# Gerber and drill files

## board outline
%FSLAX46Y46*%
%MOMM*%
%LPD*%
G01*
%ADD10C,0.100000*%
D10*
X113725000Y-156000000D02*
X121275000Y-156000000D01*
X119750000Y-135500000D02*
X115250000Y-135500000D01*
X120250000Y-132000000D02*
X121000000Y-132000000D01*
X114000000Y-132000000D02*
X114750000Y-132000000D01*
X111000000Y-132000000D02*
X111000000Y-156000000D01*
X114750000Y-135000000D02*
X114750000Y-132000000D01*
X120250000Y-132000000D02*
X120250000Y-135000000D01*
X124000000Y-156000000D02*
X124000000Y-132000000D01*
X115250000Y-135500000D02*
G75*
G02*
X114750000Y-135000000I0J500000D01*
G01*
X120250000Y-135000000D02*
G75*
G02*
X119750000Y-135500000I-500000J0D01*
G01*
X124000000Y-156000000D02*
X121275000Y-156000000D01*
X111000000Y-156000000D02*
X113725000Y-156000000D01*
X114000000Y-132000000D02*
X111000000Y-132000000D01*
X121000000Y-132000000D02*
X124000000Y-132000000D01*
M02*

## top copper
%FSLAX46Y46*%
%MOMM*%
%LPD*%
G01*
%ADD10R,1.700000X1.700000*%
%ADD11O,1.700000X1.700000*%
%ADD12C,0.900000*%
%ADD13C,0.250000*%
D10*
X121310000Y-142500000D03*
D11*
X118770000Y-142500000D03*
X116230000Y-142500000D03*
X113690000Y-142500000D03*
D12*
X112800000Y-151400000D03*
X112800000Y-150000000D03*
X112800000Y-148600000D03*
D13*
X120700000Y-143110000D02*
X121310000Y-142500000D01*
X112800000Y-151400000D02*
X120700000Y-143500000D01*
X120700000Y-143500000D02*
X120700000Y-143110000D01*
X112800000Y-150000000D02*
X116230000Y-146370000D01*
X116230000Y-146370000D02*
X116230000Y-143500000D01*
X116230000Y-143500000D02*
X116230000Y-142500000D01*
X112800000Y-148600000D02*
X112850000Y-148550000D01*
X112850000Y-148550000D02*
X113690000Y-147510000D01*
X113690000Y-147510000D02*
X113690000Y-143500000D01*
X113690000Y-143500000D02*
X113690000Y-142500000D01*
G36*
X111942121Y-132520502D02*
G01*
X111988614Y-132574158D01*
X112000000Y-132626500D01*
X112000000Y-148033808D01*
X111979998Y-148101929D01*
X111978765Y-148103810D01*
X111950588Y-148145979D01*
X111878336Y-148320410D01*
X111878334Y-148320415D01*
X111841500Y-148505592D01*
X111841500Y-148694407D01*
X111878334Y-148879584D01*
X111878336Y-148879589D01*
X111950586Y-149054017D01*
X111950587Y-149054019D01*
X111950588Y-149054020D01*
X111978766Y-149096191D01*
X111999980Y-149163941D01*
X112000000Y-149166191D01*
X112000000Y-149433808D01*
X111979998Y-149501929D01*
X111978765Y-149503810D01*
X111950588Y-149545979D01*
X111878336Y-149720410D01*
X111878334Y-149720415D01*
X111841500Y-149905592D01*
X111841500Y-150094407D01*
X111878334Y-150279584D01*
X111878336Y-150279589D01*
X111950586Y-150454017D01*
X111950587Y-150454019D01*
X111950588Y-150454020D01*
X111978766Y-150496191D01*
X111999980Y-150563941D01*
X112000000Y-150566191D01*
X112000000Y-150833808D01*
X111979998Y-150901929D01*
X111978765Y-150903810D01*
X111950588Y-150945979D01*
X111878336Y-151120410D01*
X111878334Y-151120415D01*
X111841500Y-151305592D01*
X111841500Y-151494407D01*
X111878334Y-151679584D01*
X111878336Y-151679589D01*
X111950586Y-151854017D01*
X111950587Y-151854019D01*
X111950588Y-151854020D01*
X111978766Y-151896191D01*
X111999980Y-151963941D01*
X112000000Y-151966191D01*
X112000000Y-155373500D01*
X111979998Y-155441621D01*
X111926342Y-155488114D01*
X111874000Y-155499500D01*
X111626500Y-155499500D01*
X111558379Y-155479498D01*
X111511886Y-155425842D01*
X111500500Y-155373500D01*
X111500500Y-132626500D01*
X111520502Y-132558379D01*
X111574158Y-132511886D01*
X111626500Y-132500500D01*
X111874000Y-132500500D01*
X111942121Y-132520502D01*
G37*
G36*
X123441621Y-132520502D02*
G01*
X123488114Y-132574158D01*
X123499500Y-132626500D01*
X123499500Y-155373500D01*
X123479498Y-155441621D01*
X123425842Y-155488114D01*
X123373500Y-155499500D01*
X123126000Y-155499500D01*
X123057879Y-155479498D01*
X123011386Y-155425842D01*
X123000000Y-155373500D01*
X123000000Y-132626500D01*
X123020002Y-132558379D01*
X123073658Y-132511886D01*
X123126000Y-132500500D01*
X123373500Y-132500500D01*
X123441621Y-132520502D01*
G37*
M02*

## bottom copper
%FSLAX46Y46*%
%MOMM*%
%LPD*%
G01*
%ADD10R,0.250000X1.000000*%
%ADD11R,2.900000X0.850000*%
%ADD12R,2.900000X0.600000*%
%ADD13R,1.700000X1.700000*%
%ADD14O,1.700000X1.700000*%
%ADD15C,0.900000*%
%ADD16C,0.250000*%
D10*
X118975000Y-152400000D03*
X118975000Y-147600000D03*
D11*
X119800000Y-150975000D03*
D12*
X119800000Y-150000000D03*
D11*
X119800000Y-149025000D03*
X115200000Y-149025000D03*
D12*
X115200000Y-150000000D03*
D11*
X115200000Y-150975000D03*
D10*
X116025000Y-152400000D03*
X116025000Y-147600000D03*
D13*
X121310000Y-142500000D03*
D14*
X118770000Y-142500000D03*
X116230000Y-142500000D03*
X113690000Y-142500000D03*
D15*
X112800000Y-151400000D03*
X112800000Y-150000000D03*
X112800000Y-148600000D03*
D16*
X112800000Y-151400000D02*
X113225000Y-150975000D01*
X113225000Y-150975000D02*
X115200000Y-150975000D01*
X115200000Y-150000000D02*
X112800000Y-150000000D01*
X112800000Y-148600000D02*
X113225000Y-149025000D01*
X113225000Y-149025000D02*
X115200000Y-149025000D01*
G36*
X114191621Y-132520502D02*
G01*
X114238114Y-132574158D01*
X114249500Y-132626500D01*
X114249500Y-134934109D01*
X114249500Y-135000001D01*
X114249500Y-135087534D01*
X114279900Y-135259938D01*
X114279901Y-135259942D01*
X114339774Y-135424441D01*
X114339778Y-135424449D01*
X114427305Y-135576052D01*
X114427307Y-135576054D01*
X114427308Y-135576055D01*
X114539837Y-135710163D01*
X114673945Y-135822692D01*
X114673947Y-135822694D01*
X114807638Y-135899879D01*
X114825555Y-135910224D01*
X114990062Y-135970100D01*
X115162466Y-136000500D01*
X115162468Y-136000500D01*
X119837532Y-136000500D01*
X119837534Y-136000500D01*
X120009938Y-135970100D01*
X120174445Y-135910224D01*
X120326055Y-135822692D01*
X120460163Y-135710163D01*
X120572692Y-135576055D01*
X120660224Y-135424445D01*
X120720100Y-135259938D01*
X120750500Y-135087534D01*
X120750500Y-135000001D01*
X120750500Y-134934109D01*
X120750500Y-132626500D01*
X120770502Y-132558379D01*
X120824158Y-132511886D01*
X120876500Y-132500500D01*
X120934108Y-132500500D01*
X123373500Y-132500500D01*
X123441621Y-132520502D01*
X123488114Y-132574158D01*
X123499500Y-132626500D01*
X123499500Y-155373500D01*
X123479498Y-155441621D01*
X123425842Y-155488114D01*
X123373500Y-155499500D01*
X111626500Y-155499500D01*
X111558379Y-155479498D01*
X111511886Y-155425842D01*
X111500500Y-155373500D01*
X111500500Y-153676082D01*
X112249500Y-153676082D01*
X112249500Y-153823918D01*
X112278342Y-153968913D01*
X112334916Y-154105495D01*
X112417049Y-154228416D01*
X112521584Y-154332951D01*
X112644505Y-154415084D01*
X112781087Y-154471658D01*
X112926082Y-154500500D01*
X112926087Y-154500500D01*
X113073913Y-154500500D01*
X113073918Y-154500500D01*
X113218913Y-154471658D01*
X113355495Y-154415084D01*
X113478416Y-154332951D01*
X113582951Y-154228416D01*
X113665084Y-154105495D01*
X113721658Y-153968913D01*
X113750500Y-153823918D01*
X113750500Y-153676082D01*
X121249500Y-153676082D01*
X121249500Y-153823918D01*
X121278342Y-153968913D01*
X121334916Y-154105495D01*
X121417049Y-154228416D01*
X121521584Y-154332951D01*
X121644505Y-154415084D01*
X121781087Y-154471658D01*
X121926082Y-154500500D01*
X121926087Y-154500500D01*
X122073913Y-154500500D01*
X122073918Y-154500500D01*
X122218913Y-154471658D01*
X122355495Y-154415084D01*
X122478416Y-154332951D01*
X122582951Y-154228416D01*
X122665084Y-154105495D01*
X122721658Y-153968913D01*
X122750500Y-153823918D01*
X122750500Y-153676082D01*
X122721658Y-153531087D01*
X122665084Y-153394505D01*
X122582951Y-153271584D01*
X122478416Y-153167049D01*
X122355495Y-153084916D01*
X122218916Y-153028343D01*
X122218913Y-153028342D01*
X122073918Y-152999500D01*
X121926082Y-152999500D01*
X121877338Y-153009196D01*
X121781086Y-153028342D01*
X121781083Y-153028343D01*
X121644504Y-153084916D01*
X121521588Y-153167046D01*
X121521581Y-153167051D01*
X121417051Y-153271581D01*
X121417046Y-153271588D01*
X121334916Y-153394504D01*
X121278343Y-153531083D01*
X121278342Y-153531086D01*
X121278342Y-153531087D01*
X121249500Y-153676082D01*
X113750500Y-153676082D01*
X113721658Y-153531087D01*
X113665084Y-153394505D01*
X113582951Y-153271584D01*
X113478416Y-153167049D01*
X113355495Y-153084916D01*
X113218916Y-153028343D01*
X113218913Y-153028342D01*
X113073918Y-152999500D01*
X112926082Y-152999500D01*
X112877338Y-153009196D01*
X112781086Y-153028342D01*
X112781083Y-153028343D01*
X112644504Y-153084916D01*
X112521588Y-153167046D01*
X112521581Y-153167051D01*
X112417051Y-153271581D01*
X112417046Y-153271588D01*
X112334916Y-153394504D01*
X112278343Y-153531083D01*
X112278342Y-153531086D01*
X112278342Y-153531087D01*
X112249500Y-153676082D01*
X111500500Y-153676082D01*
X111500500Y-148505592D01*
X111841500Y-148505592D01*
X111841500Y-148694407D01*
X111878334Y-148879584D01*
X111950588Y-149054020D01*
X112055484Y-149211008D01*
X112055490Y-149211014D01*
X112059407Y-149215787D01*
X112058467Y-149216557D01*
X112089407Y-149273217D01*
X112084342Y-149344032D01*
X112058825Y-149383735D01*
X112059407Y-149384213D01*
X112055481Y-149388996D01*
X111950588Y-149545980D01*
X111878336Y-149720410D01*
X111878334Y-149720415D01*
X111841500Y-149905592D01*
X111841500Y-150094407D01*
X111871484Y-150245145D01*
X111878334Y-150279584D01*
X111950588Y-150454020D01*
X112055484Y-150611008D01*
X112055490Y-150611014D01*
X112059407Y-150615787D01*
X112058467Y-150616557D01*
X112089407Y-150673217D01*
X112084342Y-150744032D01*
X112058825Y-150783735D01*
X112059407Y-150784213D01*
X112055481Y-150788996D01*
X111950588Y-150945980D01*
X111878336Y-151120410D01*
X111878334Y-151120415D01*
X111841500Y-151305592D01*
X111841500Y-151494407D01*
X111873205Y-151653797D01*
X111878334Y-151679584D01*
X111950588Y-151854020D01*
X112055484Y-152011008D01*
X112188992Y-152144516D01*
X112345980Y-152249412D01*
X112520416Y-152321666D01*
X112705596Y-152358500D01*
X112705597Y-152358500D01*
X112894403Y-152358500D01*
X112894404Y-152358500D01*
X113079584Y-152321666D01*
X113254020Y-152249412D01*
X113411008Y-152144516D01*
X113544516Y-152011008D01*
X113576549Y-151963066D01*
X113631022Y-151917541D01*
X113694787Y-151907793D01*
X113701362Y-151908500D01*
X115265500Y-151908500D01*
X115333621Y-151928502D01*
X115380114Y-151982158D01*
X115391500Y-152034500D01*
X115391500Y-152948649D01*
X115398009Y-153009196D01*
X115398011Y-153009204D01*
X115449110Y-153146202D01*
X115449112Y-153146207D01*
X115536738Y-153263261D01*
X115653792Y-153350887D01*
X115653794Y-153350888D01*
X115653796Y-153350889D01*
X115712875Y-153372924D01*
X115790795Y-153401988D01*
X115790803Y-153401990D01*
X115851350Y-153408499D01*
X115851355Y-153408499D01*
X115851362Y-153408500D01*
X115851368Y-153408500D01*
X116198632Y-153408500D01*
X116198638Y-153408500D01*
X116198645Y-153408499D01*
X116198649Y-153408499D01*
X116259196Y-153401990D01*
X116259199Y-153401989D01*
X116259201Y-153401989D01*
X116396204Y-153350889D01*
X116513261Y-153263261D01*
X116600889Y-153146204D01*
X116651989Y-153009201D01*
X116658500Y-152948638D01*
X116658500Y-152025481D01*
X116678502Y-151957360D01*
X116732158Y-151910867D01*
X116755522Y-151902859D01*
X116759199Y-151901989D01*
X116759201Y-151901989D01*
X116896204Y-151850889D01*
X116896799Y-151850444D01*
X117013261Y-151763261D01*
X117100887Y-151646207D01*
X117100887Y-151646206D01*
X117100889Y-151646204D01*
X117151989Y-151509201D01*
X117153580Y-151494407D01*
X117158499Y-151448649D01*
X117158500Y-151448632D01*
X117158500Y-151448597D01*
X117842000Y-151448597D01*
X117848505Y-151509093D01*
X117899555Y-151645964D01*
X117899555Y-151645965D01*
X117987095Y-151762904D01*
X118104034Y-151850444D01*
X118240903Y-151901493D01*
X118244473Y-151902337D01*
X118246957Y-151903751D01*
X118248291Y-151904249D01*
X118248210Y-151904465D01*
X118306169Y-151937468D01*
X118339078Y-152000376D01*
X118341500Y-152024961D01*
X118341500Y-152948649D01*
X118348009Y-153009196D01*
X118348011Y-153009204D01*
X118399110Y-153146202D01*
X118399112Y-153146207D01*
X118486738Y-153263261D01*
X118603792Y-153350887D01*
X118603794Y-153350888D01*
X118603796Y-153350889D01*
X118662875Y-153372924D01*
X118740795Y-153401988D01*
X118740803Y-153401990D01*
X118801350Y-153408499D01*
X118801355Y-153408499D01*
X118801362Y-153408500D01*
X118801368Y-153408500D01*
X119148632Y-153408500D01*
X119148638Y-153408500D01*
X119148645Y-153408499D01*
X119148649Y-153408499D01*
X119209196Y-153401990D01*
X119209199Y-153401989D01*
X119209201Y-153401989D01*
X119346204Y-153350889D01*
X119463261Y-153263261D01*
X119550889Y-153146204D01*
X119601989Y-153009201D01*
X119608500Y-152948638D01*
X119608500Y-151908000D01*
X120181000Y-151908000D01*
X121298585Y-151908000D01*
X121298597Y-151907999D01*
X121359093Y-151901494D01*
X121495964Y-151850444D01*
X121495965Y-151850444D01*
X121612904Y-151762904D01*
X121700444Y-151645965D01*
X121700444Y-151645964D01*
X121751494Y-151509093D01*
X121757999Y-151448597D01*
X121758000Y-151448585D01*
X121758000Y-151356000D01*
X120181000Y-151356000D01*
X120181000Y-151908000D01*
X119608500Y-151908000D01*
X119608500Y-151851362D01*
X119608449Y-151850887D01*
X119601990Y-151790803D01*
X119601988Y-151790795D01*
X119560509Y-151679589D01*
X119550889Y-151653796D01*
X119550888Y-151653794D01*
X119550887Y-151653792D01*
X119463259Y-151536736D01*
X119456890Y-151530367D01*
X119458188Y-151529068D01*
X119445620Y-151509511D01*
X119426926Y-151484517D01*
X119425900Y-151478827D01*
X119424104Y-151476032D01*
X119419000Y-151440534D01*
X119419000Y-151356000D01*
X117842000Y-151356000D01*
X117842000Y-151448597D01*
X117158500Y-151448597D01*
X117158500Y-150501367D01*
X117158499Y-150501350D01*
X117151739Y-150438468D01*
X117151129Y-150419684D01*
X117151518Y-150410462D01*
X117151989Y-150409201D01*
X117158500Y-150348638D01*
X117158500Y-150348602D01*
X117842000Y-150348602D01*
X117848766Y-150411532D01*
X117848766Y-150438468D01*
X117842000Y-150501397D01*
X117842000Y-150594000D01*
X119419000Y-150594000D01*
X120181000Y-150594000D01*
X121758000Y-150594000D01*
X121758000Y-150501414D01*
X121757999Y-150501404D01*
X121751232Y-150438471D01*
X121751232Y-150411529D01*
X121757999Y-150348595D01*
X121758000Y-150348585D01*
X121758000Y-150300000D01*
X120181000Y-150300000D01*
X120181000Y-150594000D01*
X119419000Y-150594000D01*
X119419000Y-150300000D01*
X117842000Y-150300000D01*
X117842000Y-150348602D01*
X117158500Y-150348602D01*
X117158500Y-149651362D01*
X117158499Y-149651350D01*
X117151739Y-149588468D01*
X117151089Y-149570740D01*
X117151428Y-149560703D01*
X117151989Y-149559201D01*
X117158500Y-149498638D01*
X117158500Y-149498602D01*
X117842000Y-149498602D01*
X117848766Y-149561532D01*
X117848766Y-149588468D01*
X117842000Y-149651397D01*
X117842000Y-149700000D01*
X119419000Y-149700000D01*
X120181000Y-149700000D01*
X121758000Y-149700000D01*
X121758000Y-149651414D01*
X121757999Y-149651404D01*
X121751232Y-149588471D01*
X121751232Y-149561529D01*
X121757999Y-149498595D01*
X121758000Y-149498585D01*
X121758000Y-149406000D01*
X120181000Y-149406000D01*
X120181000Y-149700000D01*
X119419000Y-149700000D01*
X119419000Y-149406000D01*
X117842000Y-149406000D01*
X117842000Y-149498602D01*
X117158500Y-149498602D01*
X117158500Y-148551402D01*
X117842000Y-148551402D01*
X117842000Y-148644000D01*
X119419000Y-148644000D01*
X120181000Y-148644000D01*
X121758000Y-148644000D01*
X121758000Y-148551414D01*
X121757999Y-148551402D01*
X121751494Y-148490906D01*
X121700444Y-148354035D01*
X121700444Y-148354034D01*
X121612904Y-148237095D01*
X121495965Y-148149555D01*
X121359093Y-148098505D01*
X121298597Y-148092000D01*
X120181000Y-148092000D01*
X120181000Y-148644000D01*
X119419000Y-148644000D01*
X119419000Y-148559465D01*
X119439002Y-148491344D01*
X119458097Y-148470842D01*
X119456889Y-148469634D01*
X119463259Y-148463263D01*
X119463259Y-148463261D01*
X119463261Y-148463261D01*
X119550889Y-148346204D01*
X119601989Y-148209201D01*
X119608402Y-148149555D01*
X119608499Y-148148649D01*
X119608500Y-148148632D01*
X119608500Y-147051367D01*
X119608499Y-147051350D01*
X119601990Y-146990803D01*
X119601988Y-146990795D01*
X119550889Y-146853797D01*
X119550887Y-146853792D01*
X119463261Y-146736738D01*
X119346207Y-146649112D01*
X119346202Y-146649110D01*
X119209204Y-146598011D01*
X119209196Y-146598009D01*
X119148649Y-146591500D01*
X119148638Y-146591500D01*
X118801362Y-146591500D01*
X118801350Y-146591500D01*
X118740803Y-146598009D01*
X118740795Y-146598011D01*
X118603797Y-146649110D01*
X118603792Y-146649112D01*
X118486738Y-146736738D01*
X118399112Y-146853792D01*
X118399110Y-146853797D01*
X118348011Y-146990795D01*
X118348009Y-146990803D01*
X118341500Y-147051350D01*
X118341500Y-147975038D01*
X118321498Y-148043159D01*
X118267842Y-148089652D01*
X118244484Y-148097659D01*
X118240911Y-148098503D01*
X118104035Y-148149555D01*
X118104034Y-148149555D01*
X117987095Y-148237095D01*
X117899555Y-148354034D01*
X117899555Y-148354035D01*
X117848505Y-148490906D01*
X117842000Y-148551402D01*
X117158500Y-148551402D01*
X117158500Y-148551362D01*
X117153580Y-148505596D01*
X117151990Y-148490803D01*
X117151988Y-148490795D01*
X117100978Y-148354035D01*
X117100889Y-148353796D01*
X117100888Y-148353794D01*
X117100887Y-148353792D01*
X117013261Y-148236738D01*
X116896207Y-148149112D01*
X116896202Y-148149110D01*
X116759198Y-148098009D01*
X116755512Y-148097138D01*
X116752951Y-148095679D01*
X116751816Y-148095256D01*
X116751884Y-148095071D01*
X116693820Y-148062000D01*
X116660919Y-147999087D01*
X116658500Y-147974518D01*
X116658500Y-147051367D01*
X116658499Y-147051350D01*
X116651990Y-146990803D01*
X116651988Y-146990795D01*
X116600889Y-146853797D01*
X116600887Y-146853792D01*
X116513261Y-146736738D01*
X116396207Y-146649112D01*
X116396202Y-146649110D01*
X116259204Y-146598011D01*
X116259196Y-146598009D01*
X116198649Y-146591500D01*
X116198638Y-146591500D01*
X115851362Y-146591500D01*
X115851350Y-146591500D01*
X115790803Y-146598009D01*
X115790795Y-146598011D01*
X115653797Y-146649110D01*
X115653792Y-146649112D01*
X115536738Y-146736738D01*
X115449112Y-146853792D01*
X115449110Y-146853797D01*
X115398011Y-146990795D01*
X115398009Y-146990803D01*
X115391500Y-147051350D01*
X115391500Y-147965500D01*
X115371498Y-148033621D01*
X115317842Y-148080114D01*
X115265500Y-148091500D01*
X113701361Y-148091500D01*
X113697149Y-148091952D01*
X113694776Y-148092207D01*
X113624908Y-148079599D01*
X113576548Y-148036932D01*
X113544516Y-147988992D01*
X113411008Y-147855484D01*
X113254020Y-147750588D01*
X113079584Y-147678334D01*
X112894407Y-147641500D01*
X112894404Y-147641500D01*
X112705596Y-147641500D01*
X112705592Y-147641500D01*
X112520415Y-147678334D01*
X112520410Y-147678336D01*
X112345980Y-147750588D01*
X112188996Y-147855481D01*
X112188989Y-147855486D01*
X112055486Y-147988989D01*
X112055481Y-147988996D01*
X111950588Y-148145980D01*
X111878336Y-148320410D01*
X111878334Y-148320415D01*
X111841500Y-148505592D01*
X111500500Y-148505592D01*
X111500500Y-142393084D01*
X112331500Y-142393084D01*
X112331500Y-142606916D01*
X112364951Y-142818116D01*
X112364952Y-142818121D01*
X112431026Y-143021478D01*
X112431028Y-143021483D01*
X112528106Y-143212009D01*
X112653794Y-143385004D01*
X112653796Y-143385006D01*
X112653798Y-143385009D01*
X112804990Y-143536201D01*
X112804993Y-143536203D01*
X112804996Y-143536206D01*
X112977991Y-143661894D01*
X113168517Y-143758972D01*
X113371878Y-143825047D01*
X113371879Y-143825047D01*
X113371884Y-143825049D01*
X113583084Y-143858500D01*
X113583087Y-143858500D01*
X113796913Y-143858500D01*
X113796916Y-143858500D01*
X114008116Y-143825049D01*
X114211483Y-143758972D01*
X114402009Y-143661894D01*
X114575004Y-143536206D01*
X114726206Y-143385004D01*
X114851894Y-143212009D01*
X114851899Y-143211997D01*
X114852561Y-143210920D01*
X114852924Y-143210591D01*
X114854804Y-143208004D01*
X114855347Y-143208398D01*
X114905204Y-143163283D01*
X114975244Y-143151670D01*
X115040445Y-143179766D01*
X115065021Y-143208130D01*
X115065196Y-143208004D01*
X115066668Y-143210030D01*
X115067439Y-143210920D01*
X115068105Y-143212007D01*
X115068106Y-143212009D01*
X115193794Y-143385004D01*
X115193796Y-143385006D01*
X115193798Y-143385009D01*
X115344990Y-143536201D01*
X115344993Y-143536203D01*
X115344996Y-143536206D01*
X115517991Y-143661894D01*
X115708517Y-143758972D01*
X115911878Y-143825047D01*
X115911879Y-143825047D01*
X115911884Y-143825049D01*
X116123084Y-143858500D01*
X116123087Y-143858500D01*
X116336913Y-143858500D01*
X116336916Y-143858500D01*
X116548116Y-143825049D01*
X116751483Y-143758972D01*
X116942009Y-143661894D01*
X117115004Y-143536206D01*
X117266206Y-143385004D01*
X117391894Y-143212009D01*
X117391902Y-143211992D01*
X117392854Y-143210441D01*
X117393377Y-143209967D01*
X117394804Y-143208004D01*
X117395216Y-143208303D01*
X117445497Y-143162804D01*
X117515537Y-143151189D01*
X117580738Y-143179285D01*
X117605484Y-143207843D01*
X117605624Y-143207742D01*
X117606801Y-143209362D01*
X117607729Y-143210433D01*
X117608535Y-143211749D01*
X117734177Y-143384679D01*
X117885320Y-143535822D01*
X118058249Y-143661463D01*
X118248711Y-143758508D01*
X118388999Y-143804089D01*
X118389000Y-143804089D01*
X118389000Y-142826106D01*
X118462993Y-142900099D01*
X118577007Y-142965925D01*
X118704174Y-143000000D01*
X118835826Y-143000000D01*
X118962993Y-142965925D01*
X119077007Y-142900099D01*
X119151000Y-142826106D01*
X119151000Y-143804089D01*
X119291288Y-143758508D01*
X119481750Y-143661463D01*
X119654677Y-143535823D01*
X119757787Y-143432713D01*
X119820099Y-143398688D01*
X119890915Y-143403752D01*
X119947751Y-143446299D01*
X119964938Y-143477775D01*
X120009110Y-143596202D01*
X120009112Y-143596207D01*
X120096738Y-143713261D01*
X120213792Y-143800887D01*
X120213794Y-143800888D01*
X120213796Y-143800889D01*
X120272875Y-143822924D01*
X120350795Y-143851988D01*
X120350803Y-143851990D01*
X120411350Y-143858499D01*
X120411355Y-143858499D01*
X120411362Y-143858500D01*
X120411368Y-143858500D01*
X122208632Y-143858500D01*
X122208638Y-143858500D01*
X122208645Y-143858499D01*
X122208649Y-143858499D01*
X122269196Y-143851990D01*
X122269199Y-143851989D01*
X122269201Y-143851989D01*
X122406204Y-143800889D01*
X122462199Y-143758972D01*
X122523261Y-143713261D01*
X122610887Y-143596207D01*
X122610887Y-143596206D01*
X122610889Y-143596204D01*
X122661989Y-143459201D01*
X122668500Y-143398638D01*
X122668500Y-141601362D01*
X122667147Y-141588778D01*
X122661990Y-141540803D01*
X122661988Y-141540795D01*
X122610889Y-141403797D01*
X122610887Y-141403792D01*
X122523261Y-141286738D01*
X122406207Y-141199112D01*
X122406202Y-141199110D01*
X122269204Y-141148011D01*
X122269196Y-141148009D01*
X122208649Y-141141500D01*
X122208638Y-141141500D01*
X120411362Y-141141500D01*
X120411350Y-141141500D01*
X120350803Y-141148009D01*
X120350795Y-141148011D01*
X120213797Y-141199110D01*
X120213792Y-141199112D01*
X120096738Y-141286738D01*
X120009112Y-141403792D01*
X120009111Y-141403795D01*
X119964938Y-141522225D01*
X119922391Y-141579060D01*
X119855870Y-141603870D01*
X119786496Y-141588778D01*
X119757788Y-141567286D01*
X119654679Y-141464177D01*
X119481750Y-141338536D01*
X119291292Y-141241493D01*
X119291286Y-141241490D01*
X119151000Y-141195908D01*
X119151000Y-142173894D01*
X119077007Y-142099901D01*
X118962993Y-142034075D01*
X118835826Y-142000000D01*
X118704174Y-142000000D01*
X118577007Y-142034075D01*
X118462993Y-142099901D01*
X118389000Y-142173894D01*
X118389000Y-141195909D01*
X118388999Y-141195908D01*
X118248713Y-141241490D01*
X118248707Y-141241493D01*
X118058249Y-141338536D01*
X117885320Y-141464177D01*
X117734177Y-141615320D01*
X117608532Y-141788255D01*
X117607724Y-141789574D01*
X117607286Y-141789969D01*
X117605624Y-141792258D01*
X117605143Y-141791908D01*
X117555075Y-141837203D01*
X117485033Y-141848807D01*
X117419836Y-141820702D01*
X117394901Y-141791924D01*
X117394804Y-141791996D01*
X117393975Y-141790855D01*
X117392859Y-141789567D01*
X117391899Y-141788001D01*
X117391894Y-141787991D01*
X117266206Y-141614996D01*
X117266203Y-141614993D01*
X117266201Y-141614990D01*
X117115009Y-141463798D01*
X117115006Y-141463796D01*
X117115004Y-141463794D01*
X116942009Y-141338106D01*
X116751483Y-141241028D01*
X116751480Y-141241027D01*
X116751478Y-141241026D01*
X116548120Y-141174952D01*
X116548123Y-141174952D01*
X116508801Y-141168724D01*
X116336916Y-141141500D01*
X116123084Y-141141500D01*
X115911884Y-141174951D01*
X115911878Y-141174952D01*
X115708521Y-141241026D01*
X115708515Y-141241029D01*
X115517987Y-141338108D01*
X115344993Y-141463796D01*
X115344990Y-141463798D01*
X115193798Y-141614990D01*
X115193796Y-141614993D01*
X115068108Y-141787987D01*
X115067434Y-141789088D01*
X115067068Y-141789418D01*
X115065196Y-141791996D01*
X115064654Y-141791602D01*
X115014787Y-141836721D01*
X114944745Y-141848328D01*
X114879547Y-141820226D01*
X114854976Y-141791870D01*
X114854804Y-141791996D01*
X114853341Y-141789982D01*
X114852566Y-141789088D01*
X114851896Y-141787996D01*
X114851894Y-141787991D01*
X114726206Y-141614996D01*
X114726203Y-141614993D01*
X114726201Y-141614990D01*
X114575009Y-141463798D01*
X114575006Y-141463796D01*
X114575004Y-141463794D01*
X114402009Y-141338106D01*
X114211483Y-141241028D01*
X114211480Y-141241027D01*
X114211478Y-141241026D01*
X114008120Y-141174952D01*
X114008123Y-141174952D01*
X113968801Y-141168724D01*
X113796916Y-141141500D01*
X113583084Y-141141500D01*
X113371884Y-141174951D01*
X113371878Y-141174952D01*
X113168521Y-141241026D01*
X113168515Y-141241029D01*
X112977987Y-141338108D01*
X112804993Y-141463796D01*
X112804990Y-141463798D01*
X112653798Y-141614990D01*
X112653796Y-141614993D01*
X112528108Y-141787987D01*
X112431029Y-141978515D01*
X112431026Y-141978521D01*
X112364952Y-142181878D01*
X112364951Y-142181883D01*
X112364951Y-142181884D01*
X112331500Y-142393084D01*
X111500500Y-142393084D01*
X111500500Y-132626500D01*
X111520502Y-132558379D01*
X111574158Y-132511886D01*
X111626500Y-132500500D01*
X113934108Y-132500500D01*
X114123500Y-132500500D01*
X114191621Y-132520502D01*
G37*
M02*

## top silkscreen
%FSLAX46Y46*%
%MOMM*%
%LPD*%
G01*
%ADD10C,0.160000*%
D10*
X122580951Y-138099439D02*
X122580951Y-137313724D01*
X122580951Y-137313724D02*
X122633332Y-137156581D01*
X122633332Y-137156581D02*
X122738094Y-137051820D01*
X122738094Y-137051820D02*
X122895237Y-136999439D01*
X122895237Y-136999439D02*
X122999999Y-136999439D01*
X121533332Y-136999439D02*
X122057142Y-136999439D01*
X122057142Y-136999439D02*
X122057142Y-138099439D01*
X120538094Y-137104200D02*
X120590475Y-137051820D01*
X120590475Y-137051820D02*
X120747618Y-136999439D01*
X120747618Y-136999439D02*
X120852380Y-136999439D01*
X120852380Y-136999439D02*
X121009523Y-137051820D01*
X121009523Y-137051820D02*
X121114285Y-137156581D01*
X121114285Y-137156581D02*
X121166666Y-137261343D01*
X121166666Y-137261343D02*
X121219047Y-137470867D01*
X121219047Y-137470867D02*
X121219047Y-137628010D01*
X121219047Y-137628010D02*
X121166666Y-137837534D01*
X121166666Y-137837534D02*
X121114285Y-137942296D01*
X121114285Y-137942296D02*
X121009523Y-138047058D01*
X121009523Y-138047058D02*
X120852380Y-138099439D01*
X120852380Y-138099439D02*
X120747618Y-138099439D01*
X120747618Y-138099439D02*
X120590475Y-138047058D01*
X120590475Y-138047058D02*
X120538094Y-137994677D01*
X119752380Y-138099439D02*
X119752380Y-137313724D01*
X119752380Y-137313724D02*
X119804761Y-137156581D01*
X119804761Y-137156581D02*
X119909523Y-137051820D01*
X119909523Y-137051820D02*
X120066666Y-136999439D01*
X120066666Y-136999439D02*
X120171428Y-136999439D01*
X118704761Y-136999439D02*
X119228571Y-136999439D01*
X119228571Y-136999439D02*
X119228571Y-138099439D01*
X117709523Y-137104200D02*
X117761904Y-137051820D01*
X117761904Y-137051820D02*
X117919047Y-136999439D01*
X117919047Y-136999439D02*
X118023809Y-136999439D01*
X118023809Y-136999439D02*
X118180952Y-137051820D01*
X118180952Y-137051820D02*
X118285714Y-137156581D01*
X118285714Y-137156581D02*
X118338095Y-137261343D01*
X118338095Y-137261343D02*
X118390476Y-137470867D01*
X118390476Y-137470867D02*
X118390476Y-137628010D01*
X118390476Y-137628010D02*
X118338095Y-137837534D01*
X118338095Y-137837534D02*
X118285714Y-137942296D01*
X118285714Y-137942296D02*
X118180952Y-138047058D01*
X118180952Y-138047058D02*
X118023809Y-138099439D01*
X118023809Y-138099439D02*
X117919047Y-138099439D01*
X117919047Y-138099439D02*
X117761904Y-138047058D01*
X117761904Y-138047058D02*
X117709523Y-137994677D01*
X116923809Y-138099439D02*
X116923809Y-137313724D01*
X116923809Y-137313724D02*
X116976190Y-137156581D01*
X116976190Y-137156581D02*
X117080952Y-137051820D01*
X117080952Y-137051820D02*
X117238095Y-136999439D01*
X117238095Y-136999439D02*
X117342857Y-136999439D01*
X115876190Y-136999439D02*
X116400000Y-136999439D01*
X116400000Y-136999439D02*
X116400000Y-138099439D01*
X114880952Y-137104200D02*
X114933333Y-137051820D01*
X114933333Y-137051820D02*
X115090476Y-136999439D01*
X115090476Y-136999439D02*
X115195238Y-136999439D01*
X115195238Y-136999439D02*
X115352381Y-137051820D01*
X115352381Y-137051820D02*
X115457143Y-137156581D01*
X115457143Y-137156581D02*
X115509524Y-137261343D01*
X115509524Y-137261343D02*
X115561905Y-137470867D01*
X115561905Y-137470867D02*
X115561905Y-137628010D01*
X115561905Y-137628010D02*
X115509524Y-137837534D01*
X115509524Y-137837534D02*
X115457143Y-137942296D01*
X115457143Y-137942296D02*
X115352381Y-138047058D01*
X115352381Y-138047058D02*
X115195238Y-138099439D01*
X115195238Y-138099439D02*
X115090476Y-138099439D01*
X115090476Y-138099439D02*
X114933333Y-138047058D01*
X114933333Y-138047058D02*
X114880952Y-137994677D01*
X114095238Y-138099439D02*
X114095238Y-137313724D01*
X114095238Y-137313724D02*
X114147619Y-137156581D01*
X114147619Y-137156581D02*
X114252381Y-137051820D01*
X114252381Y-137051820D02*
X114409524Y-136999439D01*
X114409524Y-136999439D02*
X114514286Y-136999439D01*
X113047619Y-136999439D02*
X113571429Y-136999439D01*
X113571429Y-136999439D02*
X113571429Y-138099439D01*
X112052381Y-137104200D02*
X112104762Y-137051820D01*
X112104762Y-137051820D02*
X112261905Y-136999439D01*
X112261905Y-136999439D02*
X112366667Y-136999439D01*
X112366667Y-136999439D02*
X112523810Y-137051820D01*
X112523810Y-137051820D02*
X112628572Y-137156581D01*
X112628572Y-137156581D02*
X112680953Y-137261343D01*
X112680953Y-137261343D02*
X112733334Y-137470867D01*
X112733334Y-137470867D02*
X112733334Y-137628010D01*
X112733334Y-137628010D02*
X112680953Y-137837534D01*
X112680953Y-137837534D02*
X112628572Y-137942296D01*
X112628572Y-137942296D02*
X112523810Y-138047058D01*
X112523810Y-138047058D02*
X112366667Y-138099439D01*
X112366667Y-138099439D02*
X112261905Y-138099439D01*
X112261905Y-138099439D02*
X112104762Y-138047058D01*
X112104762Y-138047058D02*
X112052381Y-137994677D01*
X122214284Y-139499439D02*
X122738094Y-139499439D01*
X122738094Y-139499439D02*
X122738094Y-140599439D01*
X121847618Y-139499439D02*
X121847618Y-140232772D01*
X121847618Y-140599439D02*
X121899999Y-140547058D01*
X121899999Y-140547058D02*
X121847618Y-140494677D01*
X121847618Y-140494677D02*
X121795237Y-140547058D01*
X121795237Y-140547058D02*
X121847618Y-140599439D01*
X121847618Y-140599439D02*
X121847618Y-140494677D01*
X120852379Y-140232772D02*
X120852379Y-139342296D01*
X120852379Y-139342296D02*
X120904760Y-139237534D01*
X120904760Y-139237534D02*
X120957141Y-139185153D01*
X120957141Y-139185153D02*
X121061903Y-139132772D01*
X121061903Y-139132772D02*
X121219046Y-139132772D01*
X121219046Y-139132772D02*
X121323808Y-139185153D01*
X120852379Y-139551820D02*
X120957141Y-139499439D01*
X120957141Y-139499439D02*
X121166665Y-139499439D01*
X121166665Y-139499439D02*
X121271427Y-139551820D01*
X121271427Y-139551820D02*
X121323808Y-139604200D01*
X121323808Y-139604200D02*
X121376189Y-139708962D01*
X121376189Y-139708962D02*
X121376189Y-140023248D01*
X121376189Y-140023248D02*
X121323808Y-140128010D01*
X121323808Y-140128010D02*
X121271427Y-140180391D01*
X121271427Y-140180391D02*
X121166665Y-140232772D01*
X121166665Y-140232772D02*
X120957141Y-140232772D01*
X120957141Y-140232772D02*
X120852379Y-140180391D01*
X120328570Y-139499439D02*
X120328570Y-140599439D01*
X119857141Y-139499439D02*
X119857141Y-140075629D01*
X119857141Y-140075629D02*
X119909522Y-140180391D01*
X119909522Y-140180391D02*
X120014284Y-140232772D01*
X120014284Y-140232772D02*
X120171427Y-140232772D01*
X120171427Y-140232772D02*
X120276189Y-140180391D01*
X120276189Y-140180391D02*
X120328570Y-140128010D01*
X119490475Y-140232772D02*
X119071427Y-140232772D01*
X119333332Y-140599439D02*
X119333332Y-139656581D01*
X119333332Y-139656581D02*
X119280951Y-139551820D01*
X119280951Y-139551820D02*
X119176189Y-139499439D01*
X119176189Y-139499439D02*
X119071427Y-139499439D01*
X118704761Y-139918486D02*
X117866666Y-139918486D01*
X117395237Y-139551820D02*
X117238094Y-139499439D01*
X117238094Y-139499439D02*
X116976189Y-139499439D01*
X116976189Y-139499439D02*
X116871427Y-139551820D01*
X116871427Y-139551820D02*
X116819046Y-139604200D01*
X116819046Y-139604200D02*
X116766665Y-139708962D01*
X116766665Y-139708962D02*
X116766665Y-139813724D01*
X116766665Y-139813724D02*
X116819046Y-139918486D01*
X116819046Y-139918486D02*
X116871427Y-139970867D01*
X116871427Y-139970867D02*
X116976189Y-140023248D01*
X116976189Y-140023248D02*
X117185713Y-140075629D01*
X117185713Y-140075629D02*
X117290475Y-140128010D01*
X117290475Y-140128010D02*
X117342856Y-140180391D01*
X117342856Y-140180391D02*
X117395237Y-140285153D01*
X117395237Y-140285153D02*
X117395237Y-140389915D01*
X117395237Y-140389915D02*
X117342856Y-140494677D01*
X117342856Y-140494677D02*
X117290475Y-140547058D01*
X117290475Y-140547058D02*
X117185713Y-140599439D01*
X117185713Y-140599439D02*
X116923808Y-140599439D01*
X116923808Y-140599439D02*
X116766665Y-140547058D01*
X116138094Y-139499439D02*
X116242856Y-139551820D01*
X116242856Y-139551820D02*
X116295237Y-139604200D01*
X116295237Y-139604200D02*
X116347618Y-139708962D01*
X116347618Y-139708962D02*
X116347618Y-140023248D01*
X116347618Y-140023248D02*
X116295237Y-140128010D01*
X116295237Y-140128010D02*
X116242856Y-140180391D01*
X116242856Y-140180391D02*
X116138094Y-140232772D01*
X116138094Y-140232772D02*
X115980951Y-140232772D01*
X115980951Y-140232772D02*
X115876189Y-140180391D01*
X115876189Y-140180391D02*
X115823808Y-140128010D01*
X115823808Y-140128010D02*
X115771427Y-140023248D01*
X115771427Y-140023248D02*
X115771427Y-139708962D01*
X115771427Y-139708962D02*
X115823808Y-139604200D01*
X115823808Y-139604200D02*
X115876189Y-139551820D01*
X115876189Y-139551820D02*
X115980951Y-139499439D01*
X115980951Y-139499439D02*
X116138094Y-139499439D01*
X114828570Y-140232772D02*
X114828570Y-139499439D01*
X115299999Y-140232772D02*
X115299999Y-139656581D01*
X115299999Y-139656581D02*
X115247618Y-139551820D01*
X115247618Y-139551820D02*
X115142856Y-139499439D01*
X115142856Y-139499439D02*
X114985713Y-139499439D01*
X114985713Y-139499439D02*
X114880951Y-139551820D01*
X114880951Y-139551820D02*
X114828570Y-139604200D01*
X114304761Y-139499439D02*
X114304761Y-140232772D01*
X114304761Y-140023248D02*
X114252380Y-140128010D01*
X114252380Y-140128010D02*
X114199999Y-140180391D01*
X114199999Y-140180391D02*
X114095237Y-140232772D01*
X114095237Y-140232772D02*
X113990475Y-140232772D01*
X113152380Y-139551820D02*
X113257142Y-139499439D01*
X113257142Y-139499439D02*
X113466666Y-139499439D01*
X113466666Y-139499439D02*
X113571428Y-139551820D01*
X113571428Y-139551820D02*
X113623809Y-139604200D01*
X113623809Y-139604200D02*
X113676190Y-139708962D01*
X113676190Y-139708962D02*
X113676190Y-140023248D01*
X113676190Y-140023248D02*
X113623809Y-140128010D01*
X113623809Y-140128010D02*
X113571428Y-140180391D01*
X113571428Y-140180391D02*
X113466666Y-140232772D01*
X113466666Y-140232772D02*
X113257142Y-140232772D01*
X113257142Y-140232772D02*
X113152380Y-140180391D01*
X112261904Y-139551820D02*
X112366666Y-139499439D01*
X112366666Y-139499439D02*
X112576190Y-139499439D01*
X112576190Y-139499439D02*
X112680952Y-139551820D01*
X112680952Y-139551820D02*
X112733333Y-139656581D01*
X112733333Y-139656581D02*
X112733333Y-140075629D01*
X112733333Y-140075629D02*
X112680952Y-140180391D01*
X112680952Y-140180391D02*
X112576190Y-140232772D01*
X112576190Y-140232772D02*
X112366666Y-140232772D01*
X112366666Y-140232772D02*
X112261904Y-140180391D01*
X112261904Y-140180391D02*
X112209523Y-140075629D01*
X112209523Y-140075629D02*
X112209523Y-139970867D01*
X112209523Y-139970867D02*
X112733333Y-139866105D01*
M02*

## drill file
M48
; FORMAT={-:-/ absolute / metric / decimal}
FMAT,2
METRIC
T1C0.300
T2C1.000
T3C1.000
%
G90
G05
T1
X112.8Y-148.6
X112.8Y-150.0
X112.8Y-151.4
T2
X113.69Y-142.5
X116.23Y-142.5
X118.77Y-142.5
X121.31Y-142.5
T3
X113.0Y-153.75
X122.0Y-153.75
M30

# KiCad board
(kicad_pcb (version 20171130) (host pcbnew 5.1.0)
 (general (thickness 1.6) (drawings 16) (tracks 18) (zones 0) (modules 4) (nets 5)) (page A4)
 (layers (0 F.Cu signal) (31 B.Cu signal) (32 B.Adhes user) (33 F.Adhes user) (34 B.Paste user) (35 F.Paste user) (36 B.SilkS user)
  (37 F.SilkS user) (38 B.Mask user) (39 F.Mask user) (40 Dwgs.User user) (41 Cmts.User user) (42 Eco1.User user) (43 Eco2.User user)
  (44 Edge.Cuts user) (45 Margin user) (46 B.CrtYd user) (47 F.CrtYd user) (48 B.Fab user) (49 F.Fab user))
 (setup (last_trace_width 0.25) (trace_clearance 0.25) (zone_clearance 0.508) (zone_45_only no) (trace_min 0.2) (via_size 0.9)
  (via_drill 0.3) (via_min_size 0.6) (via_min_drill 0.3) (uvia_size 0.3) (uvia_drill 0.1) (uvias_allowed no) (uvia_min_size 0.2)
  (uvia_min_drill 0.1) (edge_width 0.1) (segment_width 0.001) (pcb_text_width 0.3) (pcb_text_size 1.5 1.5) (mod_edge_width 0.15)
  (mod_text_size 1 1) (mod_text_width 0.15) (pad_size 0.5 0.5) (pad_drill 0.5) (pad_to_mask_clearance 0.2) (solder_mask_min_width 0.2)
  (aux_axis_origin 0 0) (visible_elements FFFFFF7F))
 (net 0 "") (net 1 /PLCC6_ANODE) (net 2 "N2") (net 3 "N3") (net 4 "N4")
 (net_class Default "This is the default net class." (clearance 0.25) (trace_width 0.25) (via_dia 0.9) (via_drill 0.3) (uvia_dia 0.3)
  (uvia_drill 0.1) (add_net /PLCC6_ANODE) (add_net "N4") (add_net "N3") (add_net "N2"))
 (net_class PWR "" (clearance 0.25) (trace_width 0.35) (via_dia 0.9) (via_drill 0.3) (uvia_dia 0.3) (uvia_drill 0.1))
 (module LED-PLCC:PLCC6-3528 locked (layer B.Cu) (at 117.5 150 270)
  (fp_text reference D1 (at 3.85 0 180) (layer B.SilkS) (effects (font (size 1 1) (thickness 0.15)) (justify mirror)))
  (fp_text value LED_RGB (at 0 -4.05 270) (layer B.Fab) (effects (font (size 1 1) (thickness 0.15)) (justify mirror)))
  (pad ~ smd rect (at 2.4 -1.475 270) (size 1 0.25) (layers B.Cu B.Paste B.Mask))
  (pad ~ smd rect (at -2.4 -1.475 270) (size 1 0.25) (layers B.Cu B.Paste B.Mask))
  (pad 6 smd rect (at 0.975 -2.3 270) (size 0.85 2.9) (layers B.Cu B.Paste B.Mask) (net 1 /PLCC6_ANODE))
  (pad 5 smd rect (at 0 -2.3 270) (size 0.6 2.9) (layers B.Cu B.Paste B.Mask) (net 1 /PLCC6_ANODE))
  (pad 4 smd rect (at -0.975 -2.3 270) (size 0.85 2.9) (layers B.Cu B.Paste B.Mask) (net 1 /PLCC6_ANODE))
  (pad 3 smd rect (at -0.975 2.3 270) (size 0.85 2.9) (layers B.Cu B.Paste B.Mask) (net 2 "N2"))
  (pad 2 smd rect (at 0 2.3 270) (size 0.6 2.9) (layers B.Cu B.Paste B.Mask) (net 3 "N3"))
  (pad 1 smd rect (at 0.975 2.3 270) (size 0.85 2.9) (layers B.Cu B.Paste B.Mask) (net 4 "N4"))
  (pad ~ smd rect (at 2.4 1.475 270) (size 1 0.25) (layers B.Cu B.Paste B.Mask))
  (pad ~ smd rect (at -2.4 1.475 270) (size 1 0.25) (layers B.Cu B.Paste B.Mask)))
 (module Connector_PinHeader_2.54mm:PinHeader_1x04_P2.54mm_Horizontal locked (layer B.Cu) (at 121.31 142.5 90)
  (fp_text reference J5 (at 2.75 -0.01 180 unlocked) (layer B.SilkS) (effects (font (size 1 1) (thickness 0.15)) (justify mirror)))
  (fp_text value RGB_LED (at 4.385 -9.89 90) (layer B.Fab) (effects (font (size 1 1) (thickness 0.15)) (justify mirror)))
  (pad 1 thru_hole rect (at 0 0 90) (size 1.7 1.7) (drill 1) (layers *.Cu *.Mask) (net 4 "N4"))
  (pad 2 thru_hole oval (at 0 -2.54 90) (size 1.7 1.7) (drill 1) (layers *.Cu *.Mask) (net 1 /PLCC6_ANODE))
  (pad 3 thru_hole oval (at 0 -5.08 90) (size 1.7 1.7) (drill 1) (layers *.Cu *.Mask) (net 3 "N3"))
  (pad 4 thru_hole oval (at 0 -7.62 90) (size 1.7 1.7) (drill 1) (layers *.Cu *.Mask) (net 2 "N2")))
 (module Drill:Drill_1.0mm (layer F.Cu) (at 113 153.75)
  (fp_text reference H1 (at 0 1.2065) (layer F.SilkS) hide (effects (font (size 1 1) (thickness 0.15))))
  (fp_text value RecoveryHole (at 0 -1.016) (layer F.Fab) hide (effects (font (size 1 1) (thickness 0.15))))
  (pad "" np_thru_hole circle (at 0 0) (size 1 1) (drill 1) (layers *.Cu *.Mask) (solder_mask_margin 0.0001) (clearance 0.25)))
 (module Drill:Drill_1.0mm (layer F.Cu) (at 122 153.75)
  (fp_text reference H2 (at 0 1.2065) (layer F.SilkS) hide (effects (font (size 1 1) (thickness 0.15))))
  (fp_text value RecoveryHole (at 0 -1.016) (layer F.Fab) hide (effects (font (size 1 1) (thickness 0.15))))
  (pad "" np_thru_hole circle (at 0 0) (size 1 1) (drill 1) (layers *.Cu *.Mask) (solder_mask_margin 0.0001) (clearance 0.25)))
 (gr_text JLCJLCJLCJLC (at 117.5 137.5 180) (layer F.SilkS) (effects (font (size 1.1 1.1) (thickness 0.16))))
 (gr_line (start 113.725 156) (end 121.275 156) (layer Edge.Cuts) (width 0.1))
 (gr_line (start 119.75 135.5) (end 115.25 135.5) (layer Edge.Cuts) (width 0.1))
 (gr_line (start 120.25 132) (end 121 132) (layer Edge.Cuts) (width 0.1))
 (gr_line (start 114 132) (end 114.75 132) (layer Edge.Cuts) (width 0.1))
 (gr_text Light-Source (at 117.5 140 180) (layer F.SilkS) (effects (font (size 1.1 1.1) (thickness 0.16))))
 (gr_line (start 111 132) (end 111 156) (layer Edge.Cuts) (width 0.1))
 (gr_line (start 114.75 135) (end 114.75 132) (layer Edge.Cuts) (width 0.1))
 (gr_line (start 120.25 132) (end 120.25 135) (layer Edge.Cuts) (width 0.1))
 (gr_line (start 124 156) (end 124 132) (layer Edge.Cuts) (width 0.1))
 (gr_arc (start 115.25 135) (end 114.75 135) (angle -90) (layer Edge.Cuts) (width 0.1))
 (gr_arc (start 119.75 135) (end 119.75 135.5) (angle -90) (layer Edge.Cuts) (width 0.1))
 (gr_line (start 124 156) (end 121.275 156) (layer Edge.Cuts) (width 0.1))
 (gr_line (start 111 156) (end 113.725 156) (layer Edge.Cuts) (width 0.1))
 (gr_line (start 114 132) (end 111 132) (angle 90) (layer Edge.Cuts) (width 0.1))
 (gr_line (start 121 132) (end 124 132) (angle 90) (layer Edge.Cuts) (width 0.1))
 (via (at 112.8 151.4) (size 0.9) (drill 0.3) (layers F.Cu B.Cu) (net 4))
 (segment (start 112.8 151.4) (end 113.225 150.975) (width 0.25) (layer B.Cu) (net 4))
 (segment (start 113.225 150.975) (end 115.2 150.975) (width 0.25) (layer B.Cu) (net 4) (status 800000))
 (segment (start 120.7 143.11) (end 121.31 142.5) (width 0.25) (layer F.Cu) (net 4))
 (segment (start 112.8 151.4) (end 120.7 143.5) (width 0.25) (layer F.Cu) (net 4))
 (segment (start 120.7 143.5) (end 120.7 143.11) (width 0.25) (layer F.Cu) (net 4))
 (segment (start 115.2 150) (end 112.8 150) (width 0.25) (layer B.Cu) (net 3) (status 400000))
 (via (at 112.8 150) (size 0.9) (drill 0.3) (layers F.Cu B.Cu) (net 3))
 (segment (start 112.8 150) (end 116.23 146.37) (width 0.25) (layer F.Cu) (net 3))
 (segment (start 116.23 146.37) (end 116.23 143.5) (width 0.25) (layer F.Cu) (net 3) (status 800000))
 (segment (start 116.23 143.5) (end 116.23 142.5) (width 0.25) (layer F.Cu) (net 3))
 (segment (start 112.8 148.6) (end 112.85 148.55) (width 0.25) (layer F.Cu) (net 2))
 (via (at 112.8 148.6) (size 0.9) (drill 0.3) (layers F.Cu B.Cu) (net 2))
 (segment (start 112.85 148.55) (end 113.69 147.51) (width 0.25) (layer F.Cu) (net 2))
 (segment (start 113.69 147.51) (end 113.69 143.5) (width 0.25) (layer F.Cu) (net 2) (status 800000))
 (segment (start 112.8 148.6) (end 113.225 149.025) (width 0.25) (layer B.Cu) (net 2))
 (segment (start 113.225 149.025) (end 115.2 149.025) (width 0.25) (layer B.Cu) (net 2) (status 800000))
 (segment (start 113.69 143.5) (end 113.69 142.5) (width 0.25) (layer F.Cu) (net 2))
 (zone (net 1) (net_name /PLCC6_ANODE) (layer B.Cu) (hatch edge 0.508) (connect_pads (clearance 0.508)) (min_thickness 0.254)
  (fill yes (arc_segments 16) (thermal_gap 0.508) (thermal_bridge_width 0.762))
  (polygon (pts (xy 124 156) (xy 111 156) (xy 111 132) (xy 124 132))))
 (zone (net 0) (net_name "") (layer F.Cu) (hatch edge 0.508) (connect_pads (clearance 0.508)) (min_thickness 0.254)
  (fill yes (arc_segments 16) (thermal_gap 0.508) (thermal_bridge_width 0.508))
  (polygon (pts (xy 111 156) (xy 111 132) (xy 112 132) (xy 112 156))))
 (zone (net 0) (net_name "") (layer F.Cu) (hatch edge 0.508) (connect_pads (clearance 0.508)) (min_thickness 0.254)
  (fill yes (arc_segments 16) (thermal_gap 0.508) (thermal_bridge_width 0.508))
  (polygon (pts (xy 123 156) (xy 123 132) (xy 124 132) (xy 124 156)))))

